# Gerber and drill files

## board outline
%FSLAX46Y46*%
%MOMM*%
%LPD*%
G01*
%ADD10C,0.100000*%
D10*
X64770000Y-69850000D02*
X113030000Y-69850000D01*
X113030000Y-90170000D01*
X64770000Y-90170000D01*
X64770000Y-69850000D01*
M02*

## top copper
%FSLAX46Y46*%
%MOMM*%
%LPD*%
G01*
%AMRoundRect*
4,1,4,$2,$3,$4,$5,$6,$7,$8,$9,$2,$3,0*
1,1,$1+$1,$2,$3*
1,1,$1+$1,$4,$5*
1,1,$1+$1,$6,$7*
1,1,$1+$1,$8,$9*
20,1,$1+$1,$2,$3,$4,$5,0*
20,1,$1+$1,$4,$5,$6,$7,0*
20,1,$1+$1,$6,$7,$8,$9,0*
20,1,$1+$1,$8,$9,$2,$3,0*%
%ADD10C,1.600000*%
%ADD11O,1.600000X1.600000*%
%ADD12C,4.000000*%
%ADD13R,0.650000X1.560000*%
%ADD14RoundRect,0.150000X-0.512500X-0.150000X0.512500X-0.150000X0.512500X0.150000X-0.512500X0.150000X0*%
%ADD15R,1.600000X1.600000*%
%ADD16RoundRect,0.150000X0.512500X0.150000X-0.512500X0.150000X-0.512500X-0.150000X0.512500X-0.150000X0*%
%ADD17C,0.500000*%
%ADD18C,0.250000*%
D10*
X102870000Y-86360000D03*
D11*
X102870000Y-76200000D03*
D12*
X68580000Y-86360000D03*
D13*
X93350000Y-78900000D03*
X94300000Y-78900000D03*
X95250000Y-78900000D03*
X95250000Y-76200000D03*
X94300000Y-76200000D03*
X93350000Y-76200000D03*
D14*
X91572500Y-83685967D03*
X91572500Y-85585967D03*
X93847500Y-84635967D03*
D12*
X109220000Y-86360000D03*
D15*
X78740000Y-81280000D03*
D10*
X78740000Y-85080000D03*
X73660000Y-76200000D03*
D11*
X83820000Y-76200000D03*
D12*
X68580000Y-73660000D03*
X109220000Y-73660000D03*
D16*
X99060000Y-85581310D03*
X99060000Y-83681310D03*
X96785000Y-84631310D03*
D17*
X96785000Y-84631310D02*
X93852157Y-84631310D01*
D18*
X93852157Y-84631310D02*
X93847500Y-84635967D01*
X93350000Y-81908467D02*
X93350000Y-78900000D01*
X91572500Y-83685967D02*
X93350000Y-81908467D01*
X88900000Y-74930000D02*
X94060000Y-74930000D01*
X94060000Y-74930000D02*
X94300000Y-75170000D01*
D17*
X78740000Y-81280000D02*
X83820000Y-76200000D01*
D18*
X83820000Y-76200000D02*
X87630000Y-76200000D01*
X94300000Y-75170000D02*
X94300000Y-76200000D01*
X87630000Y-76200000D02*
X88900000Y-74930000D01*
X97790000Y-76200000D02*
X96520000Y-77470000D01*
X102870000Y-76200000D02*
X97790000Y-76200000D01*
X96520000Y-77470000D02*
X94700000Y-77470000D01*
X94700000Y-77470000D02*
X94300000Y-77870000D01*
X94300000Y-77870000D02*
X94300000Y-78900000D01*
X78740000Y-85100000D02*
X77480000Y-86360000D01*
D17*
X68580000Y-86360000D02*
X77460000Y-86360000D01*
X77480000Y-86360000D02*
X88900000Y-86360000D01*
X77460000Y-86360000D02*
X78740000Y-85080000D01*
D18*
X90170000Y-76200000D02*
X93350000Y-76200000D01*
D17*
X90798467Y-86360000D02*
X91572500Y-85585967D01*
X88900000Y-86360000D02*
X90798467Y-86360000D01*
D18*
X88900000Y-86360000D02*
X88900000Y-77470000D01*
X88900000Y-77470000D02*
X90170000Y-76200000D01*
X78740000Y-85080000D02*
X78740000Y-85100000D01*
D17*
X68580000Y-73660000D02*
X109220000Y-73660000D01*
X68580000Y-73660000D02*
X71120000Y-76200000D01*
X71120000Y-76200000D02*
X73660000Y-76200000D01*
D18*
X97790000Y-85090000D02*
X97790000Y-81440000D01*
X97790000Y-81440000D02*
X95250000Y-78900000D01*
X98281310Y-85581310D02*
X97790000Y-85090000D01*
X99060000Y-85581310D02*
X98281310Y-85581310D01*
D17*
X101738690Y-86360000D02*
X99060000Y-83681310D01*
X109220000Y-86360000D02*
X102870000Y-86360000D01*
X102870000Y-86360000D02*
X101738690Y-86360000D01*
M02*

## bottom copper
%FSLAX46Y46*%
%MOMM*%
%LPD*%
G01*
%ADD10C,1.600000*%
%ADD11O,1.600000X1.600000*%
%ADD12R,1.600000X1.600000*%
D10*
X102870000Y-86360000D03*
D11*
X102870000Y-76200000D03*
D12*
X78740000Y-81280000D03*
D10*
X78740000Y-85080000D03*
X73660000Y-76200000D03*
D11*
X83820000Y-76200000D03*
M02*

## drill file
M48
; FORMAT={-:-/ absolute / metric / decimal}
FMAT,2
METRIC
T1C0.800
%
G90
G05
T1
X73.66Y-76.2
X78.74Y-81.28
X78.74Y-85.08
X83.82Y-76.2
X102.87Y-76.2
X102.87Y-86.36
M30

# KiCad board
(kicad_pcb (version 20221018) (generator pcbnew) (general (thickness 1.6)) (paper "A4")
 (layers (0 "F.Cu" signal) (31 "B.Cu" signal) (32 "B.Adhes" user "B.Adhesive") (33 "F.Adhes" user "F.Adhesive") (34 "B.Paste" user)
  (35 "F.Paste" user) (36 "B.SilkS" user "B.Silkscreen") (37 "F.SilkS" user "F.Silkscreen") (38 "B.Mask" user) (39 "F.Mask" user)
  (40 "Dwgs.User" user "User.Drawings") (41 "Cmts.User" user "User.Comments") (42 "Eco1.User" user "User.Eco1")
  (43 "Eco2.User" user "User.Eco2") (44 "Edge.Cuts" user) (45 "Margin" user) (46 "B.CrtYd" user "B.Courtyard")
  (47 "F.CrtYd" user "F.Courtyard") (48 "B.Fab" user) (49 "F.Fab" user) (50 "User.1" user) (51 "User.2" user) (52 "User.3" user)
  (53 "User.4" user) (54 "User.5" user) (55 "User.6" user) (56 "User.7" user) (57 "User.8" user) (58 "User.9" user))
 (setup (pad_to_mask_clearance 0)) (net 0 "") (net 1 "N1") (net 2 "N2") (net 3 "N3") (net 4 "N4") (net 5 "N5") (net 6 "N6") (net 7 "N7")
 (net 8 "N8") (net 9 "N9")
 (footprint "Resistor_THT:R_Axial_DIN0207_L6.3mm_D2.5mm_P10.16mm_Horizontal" (layer "F.Cu") (at 102.87 86.36 90)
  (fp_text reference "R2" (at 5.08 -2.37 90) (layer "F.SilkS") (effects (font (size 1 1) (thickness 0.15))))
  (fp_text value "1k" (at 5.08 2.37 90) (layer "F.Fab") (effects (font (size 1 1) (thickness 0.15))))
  (pad "1" thru_hole circle (at 0 0 90) (size 1.6 1.6) (drill 0.8) (layers "*.Cu" "*.Mask") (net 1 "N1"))
  (pad "2" thru_hole oval (at 10.16 0 90) (size 1.6 1.6) (drill 0.8) (layers "*.Cu" "*.Mask") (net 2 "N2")))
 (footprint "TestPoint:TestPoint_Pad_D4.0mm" (layer "F.Cu") (at 68.58 86.36)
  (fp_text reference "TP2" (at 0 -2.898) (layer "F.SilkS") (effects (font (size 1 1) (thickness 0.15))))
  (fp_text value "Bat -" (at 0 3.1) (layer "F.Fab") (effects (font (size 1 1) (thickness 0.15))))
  (pad "1" smd circle (at 0 0) (size 4 4) (layers "F.Cu" "F.Mask") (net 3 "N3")))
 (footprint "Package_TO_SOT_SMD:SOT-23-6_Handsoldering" (layer "F.Cu") (at 94.3 77.55 90)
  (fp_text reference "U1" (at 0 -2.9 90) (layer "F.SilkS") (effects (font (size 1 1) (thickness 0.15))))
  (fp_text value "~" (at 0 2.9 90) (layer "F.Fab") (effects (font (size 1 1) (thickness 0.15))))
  (pad "1" smd rect (at -1.35 -0.95 90) (size 1.56 0.65) (layers "F.Cu" "F.Paste" "F.Mask") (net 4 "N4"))
  (pad "2" smd rect (at -1.35 0 90) (size 1.56 0.65) (layers "F.Cu" "F.Paste" "F.Mask") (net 2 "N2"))
  (pad "3" smd rect (at -1.35 0.95 90) (size 1.56 0.65) (layers "F.Cu" "F.Paste" "F.Mask") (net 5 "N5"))
  (pad "4" smd rect (at 1.35 0.95 90) (size 1.56 0.65) (layers "F.Cu" "F.Paste" "F.Mask") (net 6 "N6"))
  (pad "5" smd rect (at 1.35 0 90) (size 1.56 0.65) (layers "F.Cu" "F.Paste" "F.Mask") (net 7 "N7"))
  (pad "6" smd rect (at 1.35 -0.95 90) (size 1.56 0.65) (layers "F.Cu" "F.Paste" "F.Mask") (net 3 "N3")))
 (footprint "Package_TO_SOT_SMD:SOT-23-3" (layer "F.Cu") (at 92.71 84.635967)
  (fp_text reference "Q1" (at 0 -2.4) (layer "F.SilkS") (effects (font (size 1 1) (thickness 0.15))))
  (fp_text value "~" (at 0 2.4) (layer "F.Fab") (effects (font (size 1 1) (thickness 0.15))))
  (pad "1" smd roundrect (at -1.1375 -0.95) (size 1.325 0.6) (layers "F.Cu" "F.Paste" "F.Mask") (roundrect_rratio 0.25) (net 4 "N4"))
  (pad "2" smd roundrect (at -1.1375 0.95) (size 1.325 0.6) (layers "F.Cu" "F.Paste" "F.Mask") (roundrect_rratio 0.25) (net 3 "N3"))
  (pad "3" smd roundrect (at 1.1375 0) (size 1.325 0.6) (layers "F.Cu" "F.Paste" "F.Mask") (roundrect_rratio 0.25) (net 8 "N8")))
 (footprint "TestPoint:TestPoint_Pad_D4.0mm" (layer "F.Cu") (at 109.22 86.36)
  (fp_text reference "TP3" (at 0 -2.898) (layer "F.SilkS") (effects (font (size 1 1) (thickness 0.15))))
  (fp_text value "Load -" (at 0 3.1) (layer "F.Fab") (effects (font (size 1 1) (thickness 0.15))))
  (pad "1" smd circle (at 0 0) (size 4 4) (layers "F.Cu" "F.Mask") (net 1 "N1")))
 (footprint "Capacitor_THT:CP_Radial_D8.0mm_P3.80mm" (layer "F.Cu") (at 78.74 81.28 -90)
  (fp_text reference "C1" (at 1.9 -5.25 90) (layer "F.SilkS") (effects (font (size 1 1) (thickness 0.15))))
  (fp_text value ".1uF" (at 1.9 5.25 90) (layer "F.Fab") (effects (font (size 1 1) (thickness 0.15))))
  (pad "1" thru_hole rect (at 0 0 270) (size 1.6 1.6) (drill 0.8) (layers "*.Cu" "*.Mask") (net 7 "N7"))
  (pad "2" thru_hole circle (at 3.8 0 270) (size 1.6 1.6) (drill 0.8) (layers "*.Cu" "*.Mask") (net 3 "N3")))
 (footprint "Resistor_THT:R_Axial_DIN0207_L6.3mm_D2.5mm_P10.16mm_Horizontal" (layer "F.Cu") (at 73.66 76.2)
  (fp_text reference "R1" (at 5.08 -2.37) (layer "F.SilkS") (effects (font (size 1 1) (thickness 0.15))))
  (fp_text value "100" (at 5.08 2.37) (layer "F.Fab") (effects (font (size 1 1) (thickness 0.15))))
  (pad "1" thru_hole circle (at 0 0) (size 1.6 1.6) (drill 0.8) (layers "*.Cu" "*.Mask") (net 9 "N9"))
  (pad "2" thru_hole oval (at 10.16 0) (size 1.6 1.6) (drill 0.8) (layers "*.Cu" "*.Mask") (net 7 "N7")))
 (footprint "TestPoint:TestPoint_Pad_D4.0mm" (layer "F.Cu") (at 68.58 73.66)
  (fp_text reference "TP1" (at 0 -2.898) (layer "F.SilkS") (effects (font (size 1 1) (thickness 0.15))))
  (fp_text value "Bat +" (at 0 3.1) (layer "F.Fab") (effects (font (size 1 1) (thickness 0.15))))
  (pad "1" smd circle (at 0 0) (size 4 4) (layers "F.Cu" "F.Mask") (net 9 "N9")))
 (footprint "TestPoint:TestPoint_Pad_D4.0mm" (layer "F.Cu") (at 109.22 73.66)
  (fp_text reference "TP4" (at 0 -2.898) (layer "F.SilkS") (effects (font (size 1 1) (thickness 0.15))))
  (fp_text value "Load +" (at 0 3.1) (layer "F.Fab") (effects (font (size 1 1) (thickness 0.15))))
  (pad "1" smd circle (at 0 0) (size 4 4) (layers "F.Cu" "F.Mask") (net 9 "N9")))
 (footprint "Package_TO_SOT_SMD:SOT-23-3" (layer "F.Cu") (at 97.9225 84.63131 180)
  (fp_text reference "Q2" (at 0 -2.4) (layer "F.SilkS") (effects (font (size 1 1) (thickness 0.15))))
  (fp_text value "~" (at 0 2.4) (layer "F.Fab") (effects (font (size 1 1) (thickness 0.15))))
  (pad "1" smd roundrect (at -1.1375 -0.95 180) (size 1.325 0.6) (layers "F.Cu" "F.Paste" "F.Mask") (roundrect_rratio 0.25) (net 5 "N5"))
  (pad "2" smd roundrect (at -1.1375 0.95 180) (size 1.325 0.6) (layers "F.Cu" "F.Paste" "F.Mask") (roundrect_rratio 0.25) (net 1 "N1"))
  (pad "3" smd roundrect (at 1.1375 0 180) (size 1.325 0.6) (layers "F.Cu" "F.Paste" "F.Mask") (roundrect_rratio 0.25) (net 8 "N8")))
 (gr_rect (start 64.77 69.85) (end 113.03 90.17) (stroke (width 0.1) (type default)) (fill none) (layer "Edge.Cuts"))
 (segment (start 96.785 84.63131) (end 93.852157 84.63131) (width 0.5) (layer "F.Cu") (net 8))
 (segment (start 93.852157 84.63131) (end 93.8475 84.635967) (width 0.25) (layer "F.Cu") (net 8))
 (segment (start 93.35 81.908467) (end 93.35 78.9) (width 0.25) (layer "F.Cu") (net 4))
 (segment (start 91.5725 83.685967) (end 93.35 81.908467) (width 0.25) (layer "F.Cu") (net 4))
 (segment (start 88.9 74.93) (end 94.06 74.93) (width 0.25) (layer "F.Cu") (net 7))
 (segment (start 94.06 74.93) (end 94.3 75.17) (width 0.25) (layer "F.Cu") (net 7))
 (segment (start 78.74 81.28) (end 83.82 76.2) (width 0.5) (layer "F.Cu") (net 7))
 (segment (start 83.82 76.2) (end 87.63 76.2) (width 0.25) (layer "F.Cu") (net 7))
 (segment (start 94.3 75.17) (end 94.3 76.2) (width 0.25) (layer "F.Cu") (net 7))
 (segment (start 87.63 76.2) (end 88.9 74.93) (width 0.25) (layer "F.Cu") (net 7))
 (segment (start 97.79 76.2) (end 96.52 77.47) (width 0.25) (layer "F.Cu") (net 2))
 (segment (start 102.87 76.2) (end 97.79 76.2) (width 0.25) (layer "F.Cu") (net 2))
 (segment (start 96.52 77.47) (end 94.7 77.47) (width 0.25) (layer "F.Cu") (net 2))
 (segment (start 94.7 77.47) (end 94.3 77.87) (width 0.25) (layer "F.Cu") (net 2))
 (segment (start 94.3 77.87) (end 94.3 78.9) (width 0.25) (layer "F.Cu") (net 2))
 (segment (start 78.74 85.1) (end 77.48 86.36) (width 0.25) (layer "F.Cu") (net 3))
 (segment (start 68.58 86.36) (end 77.46 86.36) (width 0.5) (layer "F.Cu") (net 3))
 (segment (start 77.48 86.36) (end 88.9 86.36) (width 0.5) (layer "F.Cu") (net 3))
 (segment (start 77.46 86.36) (end 78.74 85.08) (width 0.5) (layer "F.Cu") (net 3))
 (segment (start 90.17 76.2) (end 93.35 76.2) (width 0.25) (layer "F.Cu") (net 3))
 (segment (start 90.798467 86.36) (end 91.5725 85.585967) (width 0.5) (layer "F.Cu") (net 3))
 (segment (start 88.9 86.36) (end 90.798467 86.36) (width 0.5) (layer "F.Cu") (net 3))
 (segment (start 88.9 86.36) (end 88.9 77.47) (width 0.25) (layer "F.Cu") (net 3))
 (segment (start 88.9 77.47) (end 90.17 76.2) (width 0.25) (layer "F.Cu") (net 3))
 (segment (start 78.74 85.08) (end 78.74 85.1) (width 0.25) (layer "F.Cu") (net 3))
 (segment (start 68.58 73.66) (end 109.22 73.66) (width 0.5) (layer "F.Cu") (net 9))
 (segment (start 68.58 73.66) (end 71.12 76.2) (width 0.5) (layer "F.Cu") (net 9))
 (segment (start 71.12 76.2) (end 73.66 76.2) (width 0.5) (layer "F.Cu") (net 9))
 (segment (start 97.79 85.09) (end 97.79 81.44) (width 0.25) (layer "F.Cu") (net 5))
 (segment (start 97.79 81.44) (end 95.25 78.9) (width 0.25) (layer "F.Cu") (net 5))
 (segment (start 98.28131 85.58131) (end 97.79 85.09) (width 0.25) (layer "F.Cu") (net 5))
 (segment (start 99.06 85.58131) (end 98.28131 85.58131) (width 0.25) (layer "F.Cu") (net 5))
 (segment (start 101.73869 86.36) (end 99.06 83.68131) (width 0.5) (layer "F.Cu") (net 1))
 (segment (start 109.22 86.36) (end 102.87 86.36) (width 0.5) (layer "F.Cu") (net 1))
 (segment (start 102.87 86.36) (end 101.73869 86.36) (width 0.5) (layer "F.Cu") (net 1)))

